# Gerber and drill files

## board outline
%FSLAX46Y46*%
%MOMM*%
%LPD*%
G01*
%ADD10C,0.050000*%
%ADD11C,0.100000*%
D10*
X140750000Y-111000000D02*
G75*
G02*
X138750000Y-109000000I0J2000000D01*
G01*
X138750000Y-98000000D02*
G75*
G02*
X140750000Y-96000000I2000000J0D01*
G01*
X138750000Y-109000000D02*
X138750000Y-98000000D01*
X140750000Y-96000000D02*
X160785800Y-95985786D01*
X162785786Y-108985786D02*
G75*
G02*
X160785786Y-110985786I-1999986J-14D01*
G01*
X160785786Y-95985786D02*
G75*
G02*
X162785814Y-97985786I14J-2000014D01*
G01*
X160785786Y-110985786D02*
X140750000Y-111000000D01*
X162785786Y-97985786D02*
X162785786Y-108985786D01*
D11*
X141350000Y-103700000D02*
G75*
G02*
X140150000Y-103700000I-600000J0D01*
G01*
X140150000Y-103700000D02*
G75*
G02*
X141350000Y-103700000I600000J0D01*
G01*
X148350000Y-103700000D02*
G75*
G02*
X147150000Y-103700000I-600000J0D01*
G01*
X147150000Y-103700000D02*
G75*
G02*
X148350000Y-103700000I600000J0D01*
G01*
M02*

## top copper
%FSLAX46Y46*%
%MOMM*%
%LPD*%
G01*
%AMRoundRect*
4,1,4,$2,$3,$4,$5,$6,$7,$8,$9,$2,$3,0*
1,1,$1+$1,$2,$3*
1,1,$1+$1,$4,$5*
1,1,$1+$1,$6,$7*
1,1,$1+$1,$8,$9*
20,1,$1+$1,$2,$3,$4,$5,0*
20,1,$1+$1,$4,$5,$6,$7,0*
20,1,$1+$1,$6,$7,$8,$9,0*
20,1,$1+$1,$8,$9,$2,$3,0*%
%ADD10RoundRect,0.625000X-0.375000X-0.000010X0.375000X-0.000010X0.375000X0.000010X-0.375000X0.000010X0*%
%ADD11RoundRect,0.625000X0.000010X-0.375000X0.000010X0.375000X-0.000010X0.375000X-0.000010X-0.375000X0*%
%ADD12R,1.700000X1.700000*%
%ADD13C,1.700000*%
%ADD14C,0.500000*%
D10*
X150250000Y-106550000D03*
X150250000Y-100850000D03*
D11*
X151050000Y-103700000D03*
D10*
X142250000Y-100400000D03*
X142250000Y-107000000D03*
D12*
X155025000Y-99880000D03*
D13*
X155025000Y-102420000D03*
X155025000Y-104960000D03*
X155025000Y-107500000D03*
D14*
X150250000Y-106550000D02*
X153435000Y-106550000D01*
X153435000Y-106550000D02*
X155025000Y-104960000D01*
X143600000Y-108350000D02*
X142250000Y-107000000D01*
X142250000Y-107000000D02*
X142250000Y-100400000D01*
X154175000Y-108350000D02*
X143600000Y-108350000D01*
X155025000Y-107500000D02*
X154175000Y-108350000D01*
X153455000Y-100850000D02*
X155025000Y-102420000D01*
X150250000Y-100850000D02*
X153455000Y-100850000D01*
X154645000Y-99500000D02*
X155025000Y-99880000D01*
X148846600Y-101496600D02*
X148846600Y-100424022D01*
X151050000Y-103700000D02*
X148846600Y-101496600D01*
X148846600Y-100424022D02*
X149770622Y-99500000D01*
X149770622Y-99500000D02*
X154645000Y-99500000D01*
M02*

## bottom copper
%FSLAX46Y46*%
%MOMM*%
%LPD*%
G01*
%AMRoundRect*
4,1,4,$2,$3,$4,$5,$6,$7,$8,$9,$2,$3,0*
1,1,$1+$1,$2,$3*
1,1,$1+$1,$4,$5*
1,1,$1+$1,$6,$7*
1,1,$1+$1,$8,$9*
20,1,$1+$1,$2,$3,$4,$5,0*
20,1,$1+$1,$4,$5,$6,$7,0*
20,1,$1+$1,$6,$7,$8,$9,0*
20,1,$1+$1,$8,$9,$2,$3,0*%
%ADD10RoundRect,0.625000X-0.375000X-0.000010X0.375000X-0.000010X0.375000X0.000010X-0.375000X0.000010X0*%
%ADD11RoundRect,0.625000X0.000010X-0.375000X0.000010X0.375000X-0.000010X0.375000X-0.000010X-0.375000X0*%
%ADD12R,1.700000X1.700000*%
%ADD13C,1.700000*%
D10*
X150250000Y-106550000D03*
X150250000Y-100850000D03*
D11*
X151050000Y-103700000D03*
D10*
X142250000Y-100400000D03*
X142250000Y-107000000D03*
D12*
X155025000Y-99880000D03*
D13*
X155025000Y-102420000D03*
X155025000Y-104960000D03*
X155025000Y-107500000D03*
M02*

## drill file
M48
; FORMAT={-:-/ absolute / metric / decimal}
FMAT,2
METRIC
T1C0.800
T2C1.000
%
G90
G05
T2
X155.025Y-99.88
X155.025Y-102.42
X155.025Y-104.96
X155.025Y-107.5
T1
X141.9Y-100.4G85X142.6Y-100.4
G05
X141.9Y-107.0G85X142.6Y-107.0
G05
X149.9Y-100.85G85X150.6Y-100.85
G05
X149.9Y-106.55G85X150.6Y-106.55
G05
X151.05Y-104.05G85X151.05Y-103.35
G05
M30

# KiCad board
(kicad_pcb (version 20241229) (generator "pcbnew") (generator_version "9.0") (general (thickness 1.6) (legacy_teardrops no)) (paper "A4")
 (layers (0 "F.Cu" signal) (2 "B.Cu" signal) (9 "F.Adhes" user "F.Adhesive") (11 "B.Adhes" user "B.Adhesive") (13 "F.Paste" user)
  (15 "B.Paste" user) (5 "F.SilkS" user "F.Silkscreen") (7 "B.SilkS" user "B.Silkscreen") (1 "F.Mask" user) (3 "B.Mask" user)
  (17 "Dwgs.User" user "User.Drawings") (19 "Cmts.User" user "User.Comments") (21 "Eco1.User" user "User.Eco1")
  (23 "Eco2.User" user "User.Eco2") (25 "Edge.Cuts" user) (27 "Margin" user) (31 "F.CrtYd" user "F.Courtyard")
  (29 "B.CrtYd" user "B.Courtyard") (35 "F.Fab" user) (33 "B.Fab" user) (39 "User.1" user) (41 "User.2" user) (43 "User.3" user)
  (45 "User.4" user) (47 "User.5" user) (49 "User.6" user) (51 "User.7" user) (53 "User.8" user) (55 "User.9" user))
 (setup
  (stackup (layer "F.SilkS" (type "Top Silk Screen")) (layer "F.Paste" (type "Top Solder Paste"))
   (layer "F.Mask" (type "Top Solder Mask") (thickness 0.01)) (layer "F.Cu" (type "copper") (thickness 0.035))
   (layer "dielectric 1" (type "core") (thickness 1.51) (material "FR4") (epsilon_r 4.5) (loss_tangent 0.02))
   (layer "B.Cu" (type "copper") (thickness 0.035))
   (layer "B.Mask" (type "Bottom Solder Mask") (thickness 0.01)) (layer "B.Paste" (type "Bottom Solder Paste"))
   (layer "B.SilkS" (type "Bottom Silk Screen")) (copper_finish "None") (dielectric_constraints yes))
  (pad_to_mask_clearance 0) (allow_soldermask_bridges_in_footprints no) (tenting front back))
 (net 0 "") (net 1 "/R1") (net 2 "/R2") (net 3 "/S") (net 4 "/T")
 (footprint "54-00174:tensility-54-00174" (layer "F.Cu") (at 138.75 103.7)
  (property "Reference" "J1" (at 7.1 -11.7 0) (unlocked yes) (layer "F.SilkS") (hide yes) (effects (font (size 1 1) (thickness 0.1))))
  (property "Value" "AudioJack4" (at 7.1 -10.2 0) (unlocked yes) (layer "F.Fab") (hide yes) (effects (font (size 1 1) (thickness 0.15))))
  (fp_circle (center 2 0) (end 2.6 0) (stroke (width 0.1) (type solid)) (fill no) (layer "Edge.Cuts"))
  (fp_circle (center 9 0) (end 9.6 0) (stroke (width 0.1) (type solid)) (fill no) (layer "Edge.Cuts"))
  (pad "R1" thru_hole roundrect (at 11.5 2.85) (size 2 1.25) (drill oval 1.5 0.8) (layers "*.Cu" "*.Mask") (remove_unused_layers no)
   (roundrect_rratio 0.5) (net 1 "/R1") (thermal_bridge_angle 45))
  (pad "R2" thru_hole roundrect (at 11.5 -2.85) (size 2 1.25) (drill oval 1.5 0.8) (layers "*.Cu" "*.Mask") (remove_unused_layers no)
   (roundrect_rratio 0.5) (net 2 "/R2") (thermal_bridge_angle 45))
  (pad "S" thru_hole roundrect (at 12.3 0 90) (size 2 1.25) (drill oval 1.5 0.8) (layers "*.Cu" "*.Mask") (remove_unused_layers no)
   (roundrect_rratio 0.5) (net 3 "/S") (thermal_bridge_angle 45))
  (pad "T" thru_hole roundrect (at 3.5 -3.3) (size 2 1.25) (drill oval 1.5 0.8) (layers "*.Cu" "*.Mask") (remove_unused_layers no)
   (roundrect_rratio 0.5) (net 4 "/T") (thermal_bridge_angle 45))
  (pad "T" thru_hole roundrect (at 3.5 3.3) (size 2 1.25) (drill oval 1.5 0.8) (layers "*.Cu" "*.Mask") (remove_unused_layers no)
   (roundrect_rratio 0.5) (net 4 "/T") (thermal_bridge_angle 45)))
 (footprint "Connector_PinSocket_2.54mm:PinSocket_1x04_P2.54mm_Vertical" (layer "F.Cu") (at 155.025 99.88)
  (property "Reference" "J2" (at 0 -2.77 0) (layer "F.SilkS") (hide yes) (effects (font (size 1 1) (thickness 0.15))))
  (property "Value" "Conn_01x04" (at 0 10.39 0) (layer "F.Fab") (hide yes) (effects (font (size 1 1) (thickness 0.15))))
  (pad "1" thru_hole rect (at 0 0) (size 1.7 1.7) (drill 1) (layers "*.Cu" "*.Mask") (remove_unused_layers no) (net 3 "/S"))
  (pad "2" thru_hole circle (at 0 2.54) (size 1.7 1.7) (drill 1) (layers "*.Cu" "*.Mask") (remove_unused_layers no) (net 2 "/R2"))
  (pad "3" thru_hole circle (at 0 5.08) (size 1.7 1.7) (drill 1) (layers "*.Cu" "*.Mask") (remove_unused_layers no) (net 1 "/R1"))
  (pad "4" thru_hole circle (at 0 7.62) (size 1.7 1.7) (drill 1) (layers "*.Cu" "*.Mask") (remove_unused_layers no) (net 4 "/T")))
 (gr_arc (start 140.75 111) (mid 139.335786 110.414214) (end 138.75 109) (stroke (width 0.05) (type default)) (layer "Edge.Cuts"))
 (gr_arc (start 138.75 98) (mid 139.335786 96.585786) (end 140.75 96) (stroke (width 0.05) (type default)) (layer "Edge.Cuts"))
 (gr_line (start 138.75 109) (end 138.75 98) (stroke (width 0.05) (type default)) (layer "Edge.Cuts"))
 (gr_line (start 140.75 96) (end 160.7858 95.985786) (stroke (width 0.05) (type default)) (layer "Edge.Cuts"))
 (gr_arc (start 162.785786 108.985786) (mid 162.2 110.4) (end 160.785786 110.985786) (stroke (width 0.05) (type default))
  (layer "Edge.Cuts"))
 (gr_arc (start 160.785786 95.985786) (mid 162.2 96.571572) (end 162.785786 97.985786) (stroke (width 0.05) (type default))
  (layer "Edge.Cuts"))
 (gr_line (start 160.785786 110.985786) (end 140.75 111) (stroke (width 0.05) (type default)) (layer "Edge.Cuts"))
 (gr_line (start 162.785786 97.985786) (end 162.785786 108.985786) (stroke (width 0.05) (type default)) (layer "Edge.Cuts"))
 (segment (start 150.25 106.55) (end 153.435 106.55) (width 0.5) (layer "F.Cu") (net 1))
 (segment (start 153.435 106.55) (end 155.025 104.96) (width 0.5) (layer "F.Cu") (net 1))
 (segment (start 143.6 108.35) (end 142.25 107) (width 0.5) (layer "F.Cu") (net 4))
 (segment (start 142.25 107) (end 142.25 100.4) (width 0.5) (layer "F.Cu") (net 4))
 (segment (start 154.175 108.35) (end 143.6 108.35) (width 0.5) (layer "F.Cu") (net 4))
 (segment (start 155.025 107.5) (end 154.175 108.35) (width 0.5) (layer "F.Cu") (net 4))
 (segment (start 153.455 100.85) (end 155.025 102.42) (width 0.5) (layer "F.Cu") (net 2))
 (segment (start 150.25 100.85) (end 153.455 100.85) (width 0.5) (layer "F.Cu") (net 2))
 (segment (start 154.645 99.5) (end 155.025 99.88) (width 0.5) (layer "F.Cu") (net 3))
 (segment (start 148.8466 101.4966) (end 148.8466 100.424022) (width 0.5) (layer "F.Cu") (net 3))
 (segment (start 151.05 103.7) (end 148.8466 101.4966) (width 0.5) (layer "F.Cu") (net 3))
 (segment (start 148.8466 100.424022) (end 149.770622 99.5) (width 0.5) (layer "F.Cu") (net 3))
 (segment (start 149.770622 99.5) (end 154.645 99.5) (width 0.5) (layer "F.Cu") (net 3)))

